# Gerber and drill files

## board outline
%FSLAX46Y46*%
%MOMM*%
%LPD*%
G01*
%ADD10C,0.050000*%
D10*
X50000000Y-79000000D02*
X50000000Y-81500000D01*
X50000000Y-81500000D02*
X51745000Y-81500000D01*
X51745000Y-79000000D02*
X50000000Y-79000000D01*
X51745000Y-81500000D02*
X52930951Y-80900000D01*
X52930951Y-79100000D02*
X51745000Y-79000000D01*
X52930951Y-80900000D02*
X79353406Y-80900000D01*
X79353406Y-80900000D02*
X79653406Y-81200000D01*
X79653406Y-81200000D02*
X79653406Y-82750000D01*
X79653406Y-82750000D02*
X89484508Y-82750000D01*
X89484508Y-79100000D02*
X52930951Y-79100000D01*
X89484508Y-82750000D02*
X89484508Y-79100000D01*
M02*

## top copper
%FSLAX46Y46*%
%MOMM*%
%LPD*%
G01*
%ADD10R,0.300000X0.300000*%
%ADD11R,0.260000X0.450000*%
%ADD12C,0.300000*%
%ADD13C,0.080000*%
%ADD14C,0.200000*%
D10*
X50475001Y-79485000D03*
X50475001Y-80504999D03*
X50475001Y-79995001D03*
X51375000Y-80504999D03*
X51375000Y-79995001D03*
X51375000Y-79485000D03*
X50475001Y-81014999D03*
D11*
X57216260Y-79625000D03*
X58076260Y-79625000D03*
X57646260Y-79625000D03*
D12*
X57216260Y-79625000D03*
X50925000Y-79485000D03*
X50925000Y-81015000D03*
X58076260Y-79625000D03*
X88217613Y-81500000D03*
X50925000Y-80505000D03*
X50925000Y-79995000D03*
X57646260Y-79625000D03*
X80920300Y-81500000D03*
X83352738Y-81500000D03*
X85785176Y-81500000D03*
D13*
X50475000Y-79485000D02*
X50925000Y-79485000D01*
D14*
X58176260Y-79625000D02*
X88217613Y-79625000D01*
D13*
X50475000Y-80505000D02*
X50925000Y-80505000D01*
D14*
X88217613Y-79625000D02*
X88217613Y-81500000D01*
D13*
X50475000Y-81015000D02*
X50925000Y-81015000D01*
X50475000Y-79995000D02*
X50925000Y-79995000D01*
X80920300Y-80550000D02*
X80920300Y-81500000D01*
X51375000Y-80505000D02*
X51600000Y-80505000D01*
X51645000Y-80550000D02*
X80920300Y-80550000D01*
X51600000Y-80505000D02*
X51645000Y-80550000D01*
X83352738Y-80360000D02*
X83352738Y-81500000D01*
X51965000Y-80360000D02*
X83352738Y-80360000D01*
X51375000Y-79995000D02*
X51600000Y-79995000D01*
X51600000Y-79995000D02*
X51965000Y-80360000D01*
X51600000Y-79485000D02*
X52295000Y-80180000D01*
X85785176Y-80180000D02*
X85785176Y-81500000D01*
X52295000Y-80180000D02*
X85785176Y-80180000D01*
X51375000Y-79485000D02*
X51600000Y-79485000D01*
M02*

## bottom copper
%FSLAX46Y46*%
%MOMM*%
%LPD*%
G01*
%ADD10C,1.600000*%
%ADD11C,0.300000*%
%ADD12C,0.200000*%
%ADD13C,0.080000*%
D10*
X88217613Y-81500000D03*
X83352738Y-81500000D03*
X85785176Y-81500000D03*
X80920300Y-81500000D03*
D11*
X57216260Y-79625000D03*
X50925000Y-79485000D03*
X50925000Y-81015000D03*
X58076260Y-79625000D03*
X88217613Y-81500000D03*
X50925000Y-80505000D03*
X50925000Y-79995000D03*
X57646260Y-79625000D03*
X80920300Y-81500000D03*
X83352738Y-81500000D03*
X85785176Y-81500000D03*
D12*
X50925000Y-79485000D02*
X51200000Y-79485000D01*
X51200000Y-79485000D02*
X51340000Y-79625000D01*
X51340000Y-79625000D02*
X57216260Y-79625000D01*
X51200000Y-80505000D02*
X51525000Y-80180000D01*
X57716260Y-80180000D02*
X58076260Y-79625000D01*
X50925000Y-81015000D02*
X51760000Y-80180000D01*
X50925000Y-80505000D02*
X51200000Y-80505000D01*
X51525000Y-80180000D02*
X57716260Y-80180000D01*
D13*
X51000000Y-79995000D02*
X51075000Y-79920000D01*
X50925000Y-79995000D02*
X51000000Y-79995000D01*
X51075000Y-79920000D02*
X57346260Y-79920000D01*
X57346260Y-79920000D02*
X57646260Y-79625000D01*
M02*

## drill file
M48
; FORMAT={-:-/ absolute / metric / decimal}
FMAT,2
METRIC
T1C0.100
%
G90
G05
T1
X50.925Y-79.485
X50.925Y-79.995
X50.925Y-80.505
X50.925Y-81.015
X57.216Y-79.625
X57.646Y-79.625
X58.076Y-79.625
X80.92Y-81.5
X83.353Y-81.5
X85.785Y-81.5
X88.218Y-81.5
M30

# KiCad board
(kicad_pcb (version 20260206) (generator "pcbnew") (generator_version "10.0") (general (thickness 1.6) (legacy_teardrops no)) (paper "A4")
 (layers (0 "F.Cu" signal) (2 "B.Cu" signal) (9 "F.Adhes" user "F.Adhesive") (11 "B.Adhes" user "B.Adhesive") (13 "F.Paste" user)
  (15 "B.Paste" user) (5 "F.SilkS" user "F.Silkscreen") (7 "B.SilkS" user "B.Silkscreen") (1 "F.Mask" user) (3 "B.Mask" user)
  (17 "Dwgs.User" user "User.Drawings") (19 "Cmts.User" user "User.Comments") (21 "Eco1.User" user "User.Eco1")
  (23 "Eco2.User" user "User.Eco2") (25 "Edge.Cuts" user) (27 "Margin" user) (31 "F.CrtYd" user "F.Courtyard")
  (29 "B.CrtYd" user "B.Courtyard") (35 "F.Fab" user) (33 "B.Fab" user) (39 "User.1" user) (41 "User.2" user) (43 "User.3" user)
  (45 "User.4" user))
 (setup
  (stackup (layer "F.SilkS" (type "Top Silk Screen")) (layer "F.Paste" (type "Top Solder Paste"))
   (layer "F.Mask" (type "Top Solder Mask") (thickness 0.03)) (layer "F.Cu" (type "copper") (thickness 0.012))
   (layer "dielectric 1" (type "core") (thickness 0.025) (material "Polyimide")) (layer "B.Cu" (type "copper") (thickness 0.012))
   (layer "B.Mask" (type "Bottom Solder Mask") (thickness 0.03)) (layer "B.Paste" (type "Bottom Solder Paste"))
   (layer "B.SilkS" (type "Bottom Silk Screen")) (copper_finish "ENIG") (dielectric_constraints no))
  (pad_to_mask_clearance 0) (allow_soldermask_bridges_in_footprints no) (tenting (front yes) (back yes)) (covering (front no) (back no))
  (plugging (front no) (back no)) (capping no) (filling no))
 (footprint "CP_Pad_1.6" (layer "F.Cu") (at 83.352738 81.5)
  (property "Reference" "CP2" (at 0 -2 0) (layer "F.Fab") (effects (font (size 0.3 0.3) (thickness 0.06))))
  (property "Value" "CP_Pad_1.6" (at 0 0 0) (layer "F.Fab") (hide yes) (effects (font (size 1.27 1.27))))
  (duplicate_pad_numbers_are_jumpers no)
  (pad "1" smd circle (at 0 0) (size 1.6 1.6) (layers "B.Cu" "B.Mask") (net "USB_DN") (solder_mask_margin 0.1)))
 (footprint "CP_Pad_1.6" (layer "F.Cu") (at 80.9203 81.5)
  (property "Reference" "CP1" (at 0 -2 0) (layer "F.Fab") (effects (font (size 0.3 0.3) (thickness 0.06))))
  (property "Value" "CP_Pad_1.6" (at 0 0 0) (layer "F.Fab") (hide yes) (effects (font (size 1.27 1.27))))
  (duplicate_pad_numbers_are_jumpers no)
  (pad "1" smd circle (at 0 0) (size 1.6 1.6) (layers "B.Cu" "B.Mask") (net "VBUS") (solder_mask_margin 0.1)))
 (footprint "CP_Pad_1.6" (layer "F.Cu") (at 85.785176 81.5)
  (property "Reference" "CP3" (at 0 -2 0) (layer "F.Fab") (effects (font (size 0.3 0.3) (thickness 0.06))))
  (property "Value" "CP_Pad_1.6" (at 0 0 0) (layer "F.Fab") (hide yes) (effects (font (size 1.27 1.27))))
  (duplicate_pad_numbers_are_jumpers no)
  (pad "1" smd circle (at 0 0) (size 1.6 1.6) (layers "B.Cu" "B.Mask") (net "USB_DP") (solder_mask_margin 0.1)))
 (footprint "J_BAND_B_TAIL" (layer "F.Cu") (at 50.9 80.25)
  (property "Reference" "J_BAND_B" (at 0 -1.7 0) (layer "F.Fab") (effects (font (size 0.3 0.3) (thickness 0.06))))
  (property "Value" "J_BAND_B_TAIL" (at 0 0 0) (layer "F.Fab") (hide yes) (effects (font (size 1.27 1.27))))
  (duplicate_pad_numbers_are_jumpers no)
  (pad "1" smd rect (at -0.424999 -0.765) (size 0.3 0.3) (layers "F.Cu" "F.Mask") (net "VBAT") (solder_mask_margin 0.05)
   (thermal_bridge_angle 45))
  (pad "2" smd rect (at -0.424999 0.254999) (size 0.3 0.3) (layers "F.Cu" "F.Mask") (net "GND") (solder_mask_margin 0.05)
   (thermal_bridge_angle 45))
  (pad "3" smd rect (at -0.424999 -0.254999) (size 0.3 0.3) (layers "F.Cu" "F.Mask") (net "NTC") (solder_mask_margin 0.05)
   (thermal_bridge_angle 45))
  (pad "4" smd rect (at 0.475 0.254999) (size 0.3 0.3) (layers "F.Cu" "F.Mask") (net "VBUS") (solder_mask_margin 0.05)
   (thermal_bridge_angle 45))
  (pad "5" smd rect (at 0.475 -0.254999) (size 0.3 0.3) (layers "F.Cu" "F.Mask") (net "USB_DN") (solder_mask_margin 0.05)
   (thermal_bridge_angle 45))
  (pad "6" smd rect (at 0.475 -0.765) (size 0.3 0.3) (layers "F.Cu" "F.Mask") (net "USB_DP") (solder_mask_margin 0.05)
   (thermal_bridge_angle 45))
  (pad "7" smd rect (at -0.424999 0.764999) (size 0.3 0.3) (layers "F.Cu" "F.Mask") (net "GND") (solder_mask_margin 0.05)
   (thermal_bridge_angle 45)))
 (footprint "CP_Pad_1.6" (layer "F.Cu") (at 88.217613 81.5)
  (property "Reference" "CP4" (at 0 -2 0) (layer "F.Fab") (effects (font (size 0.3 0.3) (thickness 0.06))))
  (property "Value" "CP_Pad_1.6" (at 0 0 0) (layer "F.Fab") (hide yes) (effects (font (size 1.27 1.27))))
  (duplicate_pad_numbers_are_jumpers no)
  (pad "1" smd circle (at 0 0) (size 1.6 1.6) (layers "B.Cu" "B.Mask") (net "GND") (solder_mask_margin 0.1)))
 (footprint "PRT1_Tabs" (layer "F.Cu") (at 57.64626 79.625)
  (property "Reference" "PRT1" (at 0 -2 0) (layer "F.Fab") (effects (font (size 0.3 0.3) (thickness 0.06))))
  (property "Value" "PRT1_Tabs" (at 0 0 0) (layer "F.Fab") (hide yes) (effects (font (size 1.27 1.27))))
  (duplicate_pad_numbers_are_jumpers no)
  (pad "1" smd rect (at -0.43 0) (size 0.26 0.45) (layers "F.Cu" "F.Mask") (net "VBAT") (solder_mask_margin 0.05) (thermal_bridge_angle 45))
  (pad "2" smd rect (at 0.43 0) (size 0.26 0.45) (layers "F.Cu" "F.Mask") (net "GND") (solder_mask_margin 0.05) (thermal_bridge_angle 45))
  (pad "3" smd rect (at 0 0) (size 0.26 0.45) (layers "F.Cu" "F.Mask") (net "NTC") (solder_mask_margin 0.05) (thermal_bridge_angle 45)))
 (gr_line (start 50 79) (end 50 81.5) (stroke (width 0.05) (type default)) (layer "Edge.Cuts"))
 (gr_line (start 50 81.5) (end 51.745 81.5) (stroke (width 0.05) (type default)) (layer "Edge.Cuts"))
 (gr_line (start 51.745 79) (end 50 79) (stroke (width 0.05) (type default)) (layer "Edge.Cuts"))
 (gr_line (start 51.745 81.5) (end 52.930951 80.9) (stroke (width 0.05) (type default)) (layer "Edge.Cuts"))
 (gr_line (start 52.930951 79.1) (end 51.745 79) (stroke (width 0.05) (type default)) (layer "Edge.Cuts"))
 (gr_line (start 52.930951 80.9) (end 79.353406 80.9) (stroke (width 0.05) (type default)) (layer "Edge.Cuts"))
 (gr_line (start 79.353406 80.9) (end 79.653406 81.2) (stroke (width 0.05) (type default)) (layer "Edge.Cuts"))
 (gr_line (start 79.653406 81.2) (end 79.653406 82.75) (stroke (width 0.05) (type default)) (layer "Edge.Cuts"))
 (gr_line (start 79.653406 82.75) (end 89.484508 82.75) (stroke (width 0.05) (type default)) (layer "Edge.Cuts"))
 (gr_line (start 89.484508 79.1) (end 52.930951 79.1) (stroke (width 0.05) (type default)) (layer "Edge.Cuts"))
 (gr_line (start 89.484508 82.75) (end 89.484508 79.1) (stroke (width 0.05) (type default)) (layer "Edge.Cuts"))
 (segment (start 50.475 79.485) (end 50.925 79.485) (width 0.08) (layer "F.Cu") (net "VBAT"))
 (via (at 50.925 79.485) (size 0.3) (drill 0.1) (layers "F.Cu" "B.Cu") (tenting (front yes) (back yes)) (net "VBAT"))
 (via (at 57.21626 79.625) (size 0.3) (drill 0.1) (layers "F.Cu" "B.Cu") (tenting (front yes) (back yes)) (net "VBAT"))
 (segment (start 51.2 79.485) (end 51.34 79.625) (width 0.2) (layer "B.Cu") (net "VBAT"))
 (segment (start 50.925 79.485) (end 51.2 79.485) (width 0.2) (layer "B.Cu") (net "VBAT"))
 (segment (start 51.34 79.625) (end 57.21626 79.625) (width 0.2) (layer "B.Cu") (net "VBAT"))
 (segment (start 50.475 80.505) (end 50.925 80.505) (width 0.08) (layer "F.Cu") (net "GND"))
 (segment (start 58.17626 79.625) (end 88.217613 79.625) (width 0.2) (layer "F.Cu") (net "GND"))
 (segment (start 50.475 81.015) (end 50.925 81.015) (width 0.08) (layer "F.Cu") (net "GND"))
 (segment (start 88.217613 79.625) (end 88.217613 81.5) (width 0.2) (layer "F.Cu") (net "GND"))
 (via (at 50.925 81.015) (size 0.3) (drill 0.1) (layers "F.Cu" "B.Cu") (tenting (front yes) (back yes)) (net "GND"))
 (via (at 88.217613 81.5) (size 0.3) (drill 0.1) (layers "F.Cu" "B.Cu") (tenting (front yes) (back yes)) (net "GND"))
 (via (at 50.925 80.505) (size 0.3) (drill 0.1) (layers "F.Cu" "B.Cu") (tenting (front yes) (back yes)) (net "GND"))
 (via (at 58.07626 79.625) (size 0.3) (drill 0.1) (layers "F.Cu" "B.Cu") (tenting (front yes) (back yes)) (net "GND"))
 (segment (start 50.925 81.015) (end 51.76 80.18) (width 0.2) (layer "B.Cu") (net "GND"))
 (segment (start 51.2 80.505) (end 51.525 80.18) (width 0.2) (layer "B.Cu") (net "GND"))
 (segment (start 51.525 80.18) (end 57.71626 80.18) (width 0.2) (layer "B.Cu") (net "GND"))
 (segment (start 50.925 80.505) (end 51.2 80.505) (width 0.2) (layer "B.Cu") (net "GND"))
 (segment (start 57.71626 80.18) (end 58.07626 79.625) (width 0.2) (layer "B.Cu") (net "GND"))
 (segment (start 50.475 79.995) (end 50.925 79.995) (width 0.08) (layer "F.Cu") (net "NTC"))
 (via (at 57.64626 79.625) (size 0.3) (drill 0.1) (layers "F.Cu" "B.Cu") (tenting (front yes) (back yes)) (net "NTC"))
 (via (at 50.925 79.995) (size 0.3) (drill 0.1) (layers "F.Cu" "B.Cu") (tenting (front yes) (back yes)) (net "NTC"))
 (segment (start 57.34626 79.92) (end 57.64626 79.625) (width 0.08) (layer "B.Cu") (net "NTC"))
 (segment (start 51.075 79.92) (end 57.34626 79.92) (width 0.08) (layer "B.Cu") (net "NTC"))
 (segment (start 50.925 79.995) (end 51 79.995) (width 0.08) (layer "B.Cu") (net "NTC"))
 (segment (start 51 79.995) (end 51.075 79.92) (width 0.08) (layer "B.Cu") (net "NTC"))
 (segment (start 51.6 80.505) (end 51.645 80.55) (width 0.08) (layer "F.Cu") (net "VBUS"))
 (segment (start 51.645 80.55) (end 80.9203 80.55) (width 0.08) (layer "F.Cu") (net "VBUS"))
 (segment (start 80.9203 80.55) (end 80.9203 81.5) (width 0.08) (layer "F.Cu") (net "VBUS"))
 (segment (start 51.375 80.505) (end 51.6 80.505) (width 0.08) (layer "F.Cu") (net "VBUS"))
 (via (at 80.9203 81.5) (size 0.3) (drill 0.1) (layers "F.Cu" "B.Cu") (tenting (front yes) (back yes)) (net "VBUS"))
 (segment (start 51.6 79.995) (end 51.965 80.36) (width 0.08) (layer "F.Cu") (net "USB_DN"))
 (segment (start 51.965 80.36) (end 83.352738 80.36) (width 0.08) (layer "F.Cu") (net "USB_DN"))
 (segment (start 51.375 79.995) (end 51.6 79.995) (width 0.08) (layer "F.Cu") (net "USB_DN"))
 (segment (start 83.352738 80.36) (end 83.352738 81.5) (width 0.08) (layer "F.Cu") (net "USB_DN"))
 (via (at 83.352738 81.5) (size 0.3) (drill 0.1) (layers "F.Cu" "B.Cu") (tenting (front yes) (back yes)) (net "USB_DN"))
 (segment (start 51.6 79.485) (end 52.295 80.18) (width 0.08) (layer "F.Cu") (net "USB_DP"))
 (segment (start 52.295 80.18) (end 85.785176 80.18) (width 0.08) (layer "F.Cu") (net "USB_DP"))
 (segment (start 85.785176 80.18) (end 85.785176 81.5) (width 0.08) (layer "F.Cu") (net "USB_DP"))
 (segment (start 51.375 79.485) (end 51.6 79.485) (width 0.08) (layer "F.Cu") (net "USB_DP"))
 (via (at 85.785176 81.5) (size 0.3) (drill 0.1) (layers "F.Cu" "B.Cu") (tenting (front yes) (back yes)) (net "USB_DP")))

